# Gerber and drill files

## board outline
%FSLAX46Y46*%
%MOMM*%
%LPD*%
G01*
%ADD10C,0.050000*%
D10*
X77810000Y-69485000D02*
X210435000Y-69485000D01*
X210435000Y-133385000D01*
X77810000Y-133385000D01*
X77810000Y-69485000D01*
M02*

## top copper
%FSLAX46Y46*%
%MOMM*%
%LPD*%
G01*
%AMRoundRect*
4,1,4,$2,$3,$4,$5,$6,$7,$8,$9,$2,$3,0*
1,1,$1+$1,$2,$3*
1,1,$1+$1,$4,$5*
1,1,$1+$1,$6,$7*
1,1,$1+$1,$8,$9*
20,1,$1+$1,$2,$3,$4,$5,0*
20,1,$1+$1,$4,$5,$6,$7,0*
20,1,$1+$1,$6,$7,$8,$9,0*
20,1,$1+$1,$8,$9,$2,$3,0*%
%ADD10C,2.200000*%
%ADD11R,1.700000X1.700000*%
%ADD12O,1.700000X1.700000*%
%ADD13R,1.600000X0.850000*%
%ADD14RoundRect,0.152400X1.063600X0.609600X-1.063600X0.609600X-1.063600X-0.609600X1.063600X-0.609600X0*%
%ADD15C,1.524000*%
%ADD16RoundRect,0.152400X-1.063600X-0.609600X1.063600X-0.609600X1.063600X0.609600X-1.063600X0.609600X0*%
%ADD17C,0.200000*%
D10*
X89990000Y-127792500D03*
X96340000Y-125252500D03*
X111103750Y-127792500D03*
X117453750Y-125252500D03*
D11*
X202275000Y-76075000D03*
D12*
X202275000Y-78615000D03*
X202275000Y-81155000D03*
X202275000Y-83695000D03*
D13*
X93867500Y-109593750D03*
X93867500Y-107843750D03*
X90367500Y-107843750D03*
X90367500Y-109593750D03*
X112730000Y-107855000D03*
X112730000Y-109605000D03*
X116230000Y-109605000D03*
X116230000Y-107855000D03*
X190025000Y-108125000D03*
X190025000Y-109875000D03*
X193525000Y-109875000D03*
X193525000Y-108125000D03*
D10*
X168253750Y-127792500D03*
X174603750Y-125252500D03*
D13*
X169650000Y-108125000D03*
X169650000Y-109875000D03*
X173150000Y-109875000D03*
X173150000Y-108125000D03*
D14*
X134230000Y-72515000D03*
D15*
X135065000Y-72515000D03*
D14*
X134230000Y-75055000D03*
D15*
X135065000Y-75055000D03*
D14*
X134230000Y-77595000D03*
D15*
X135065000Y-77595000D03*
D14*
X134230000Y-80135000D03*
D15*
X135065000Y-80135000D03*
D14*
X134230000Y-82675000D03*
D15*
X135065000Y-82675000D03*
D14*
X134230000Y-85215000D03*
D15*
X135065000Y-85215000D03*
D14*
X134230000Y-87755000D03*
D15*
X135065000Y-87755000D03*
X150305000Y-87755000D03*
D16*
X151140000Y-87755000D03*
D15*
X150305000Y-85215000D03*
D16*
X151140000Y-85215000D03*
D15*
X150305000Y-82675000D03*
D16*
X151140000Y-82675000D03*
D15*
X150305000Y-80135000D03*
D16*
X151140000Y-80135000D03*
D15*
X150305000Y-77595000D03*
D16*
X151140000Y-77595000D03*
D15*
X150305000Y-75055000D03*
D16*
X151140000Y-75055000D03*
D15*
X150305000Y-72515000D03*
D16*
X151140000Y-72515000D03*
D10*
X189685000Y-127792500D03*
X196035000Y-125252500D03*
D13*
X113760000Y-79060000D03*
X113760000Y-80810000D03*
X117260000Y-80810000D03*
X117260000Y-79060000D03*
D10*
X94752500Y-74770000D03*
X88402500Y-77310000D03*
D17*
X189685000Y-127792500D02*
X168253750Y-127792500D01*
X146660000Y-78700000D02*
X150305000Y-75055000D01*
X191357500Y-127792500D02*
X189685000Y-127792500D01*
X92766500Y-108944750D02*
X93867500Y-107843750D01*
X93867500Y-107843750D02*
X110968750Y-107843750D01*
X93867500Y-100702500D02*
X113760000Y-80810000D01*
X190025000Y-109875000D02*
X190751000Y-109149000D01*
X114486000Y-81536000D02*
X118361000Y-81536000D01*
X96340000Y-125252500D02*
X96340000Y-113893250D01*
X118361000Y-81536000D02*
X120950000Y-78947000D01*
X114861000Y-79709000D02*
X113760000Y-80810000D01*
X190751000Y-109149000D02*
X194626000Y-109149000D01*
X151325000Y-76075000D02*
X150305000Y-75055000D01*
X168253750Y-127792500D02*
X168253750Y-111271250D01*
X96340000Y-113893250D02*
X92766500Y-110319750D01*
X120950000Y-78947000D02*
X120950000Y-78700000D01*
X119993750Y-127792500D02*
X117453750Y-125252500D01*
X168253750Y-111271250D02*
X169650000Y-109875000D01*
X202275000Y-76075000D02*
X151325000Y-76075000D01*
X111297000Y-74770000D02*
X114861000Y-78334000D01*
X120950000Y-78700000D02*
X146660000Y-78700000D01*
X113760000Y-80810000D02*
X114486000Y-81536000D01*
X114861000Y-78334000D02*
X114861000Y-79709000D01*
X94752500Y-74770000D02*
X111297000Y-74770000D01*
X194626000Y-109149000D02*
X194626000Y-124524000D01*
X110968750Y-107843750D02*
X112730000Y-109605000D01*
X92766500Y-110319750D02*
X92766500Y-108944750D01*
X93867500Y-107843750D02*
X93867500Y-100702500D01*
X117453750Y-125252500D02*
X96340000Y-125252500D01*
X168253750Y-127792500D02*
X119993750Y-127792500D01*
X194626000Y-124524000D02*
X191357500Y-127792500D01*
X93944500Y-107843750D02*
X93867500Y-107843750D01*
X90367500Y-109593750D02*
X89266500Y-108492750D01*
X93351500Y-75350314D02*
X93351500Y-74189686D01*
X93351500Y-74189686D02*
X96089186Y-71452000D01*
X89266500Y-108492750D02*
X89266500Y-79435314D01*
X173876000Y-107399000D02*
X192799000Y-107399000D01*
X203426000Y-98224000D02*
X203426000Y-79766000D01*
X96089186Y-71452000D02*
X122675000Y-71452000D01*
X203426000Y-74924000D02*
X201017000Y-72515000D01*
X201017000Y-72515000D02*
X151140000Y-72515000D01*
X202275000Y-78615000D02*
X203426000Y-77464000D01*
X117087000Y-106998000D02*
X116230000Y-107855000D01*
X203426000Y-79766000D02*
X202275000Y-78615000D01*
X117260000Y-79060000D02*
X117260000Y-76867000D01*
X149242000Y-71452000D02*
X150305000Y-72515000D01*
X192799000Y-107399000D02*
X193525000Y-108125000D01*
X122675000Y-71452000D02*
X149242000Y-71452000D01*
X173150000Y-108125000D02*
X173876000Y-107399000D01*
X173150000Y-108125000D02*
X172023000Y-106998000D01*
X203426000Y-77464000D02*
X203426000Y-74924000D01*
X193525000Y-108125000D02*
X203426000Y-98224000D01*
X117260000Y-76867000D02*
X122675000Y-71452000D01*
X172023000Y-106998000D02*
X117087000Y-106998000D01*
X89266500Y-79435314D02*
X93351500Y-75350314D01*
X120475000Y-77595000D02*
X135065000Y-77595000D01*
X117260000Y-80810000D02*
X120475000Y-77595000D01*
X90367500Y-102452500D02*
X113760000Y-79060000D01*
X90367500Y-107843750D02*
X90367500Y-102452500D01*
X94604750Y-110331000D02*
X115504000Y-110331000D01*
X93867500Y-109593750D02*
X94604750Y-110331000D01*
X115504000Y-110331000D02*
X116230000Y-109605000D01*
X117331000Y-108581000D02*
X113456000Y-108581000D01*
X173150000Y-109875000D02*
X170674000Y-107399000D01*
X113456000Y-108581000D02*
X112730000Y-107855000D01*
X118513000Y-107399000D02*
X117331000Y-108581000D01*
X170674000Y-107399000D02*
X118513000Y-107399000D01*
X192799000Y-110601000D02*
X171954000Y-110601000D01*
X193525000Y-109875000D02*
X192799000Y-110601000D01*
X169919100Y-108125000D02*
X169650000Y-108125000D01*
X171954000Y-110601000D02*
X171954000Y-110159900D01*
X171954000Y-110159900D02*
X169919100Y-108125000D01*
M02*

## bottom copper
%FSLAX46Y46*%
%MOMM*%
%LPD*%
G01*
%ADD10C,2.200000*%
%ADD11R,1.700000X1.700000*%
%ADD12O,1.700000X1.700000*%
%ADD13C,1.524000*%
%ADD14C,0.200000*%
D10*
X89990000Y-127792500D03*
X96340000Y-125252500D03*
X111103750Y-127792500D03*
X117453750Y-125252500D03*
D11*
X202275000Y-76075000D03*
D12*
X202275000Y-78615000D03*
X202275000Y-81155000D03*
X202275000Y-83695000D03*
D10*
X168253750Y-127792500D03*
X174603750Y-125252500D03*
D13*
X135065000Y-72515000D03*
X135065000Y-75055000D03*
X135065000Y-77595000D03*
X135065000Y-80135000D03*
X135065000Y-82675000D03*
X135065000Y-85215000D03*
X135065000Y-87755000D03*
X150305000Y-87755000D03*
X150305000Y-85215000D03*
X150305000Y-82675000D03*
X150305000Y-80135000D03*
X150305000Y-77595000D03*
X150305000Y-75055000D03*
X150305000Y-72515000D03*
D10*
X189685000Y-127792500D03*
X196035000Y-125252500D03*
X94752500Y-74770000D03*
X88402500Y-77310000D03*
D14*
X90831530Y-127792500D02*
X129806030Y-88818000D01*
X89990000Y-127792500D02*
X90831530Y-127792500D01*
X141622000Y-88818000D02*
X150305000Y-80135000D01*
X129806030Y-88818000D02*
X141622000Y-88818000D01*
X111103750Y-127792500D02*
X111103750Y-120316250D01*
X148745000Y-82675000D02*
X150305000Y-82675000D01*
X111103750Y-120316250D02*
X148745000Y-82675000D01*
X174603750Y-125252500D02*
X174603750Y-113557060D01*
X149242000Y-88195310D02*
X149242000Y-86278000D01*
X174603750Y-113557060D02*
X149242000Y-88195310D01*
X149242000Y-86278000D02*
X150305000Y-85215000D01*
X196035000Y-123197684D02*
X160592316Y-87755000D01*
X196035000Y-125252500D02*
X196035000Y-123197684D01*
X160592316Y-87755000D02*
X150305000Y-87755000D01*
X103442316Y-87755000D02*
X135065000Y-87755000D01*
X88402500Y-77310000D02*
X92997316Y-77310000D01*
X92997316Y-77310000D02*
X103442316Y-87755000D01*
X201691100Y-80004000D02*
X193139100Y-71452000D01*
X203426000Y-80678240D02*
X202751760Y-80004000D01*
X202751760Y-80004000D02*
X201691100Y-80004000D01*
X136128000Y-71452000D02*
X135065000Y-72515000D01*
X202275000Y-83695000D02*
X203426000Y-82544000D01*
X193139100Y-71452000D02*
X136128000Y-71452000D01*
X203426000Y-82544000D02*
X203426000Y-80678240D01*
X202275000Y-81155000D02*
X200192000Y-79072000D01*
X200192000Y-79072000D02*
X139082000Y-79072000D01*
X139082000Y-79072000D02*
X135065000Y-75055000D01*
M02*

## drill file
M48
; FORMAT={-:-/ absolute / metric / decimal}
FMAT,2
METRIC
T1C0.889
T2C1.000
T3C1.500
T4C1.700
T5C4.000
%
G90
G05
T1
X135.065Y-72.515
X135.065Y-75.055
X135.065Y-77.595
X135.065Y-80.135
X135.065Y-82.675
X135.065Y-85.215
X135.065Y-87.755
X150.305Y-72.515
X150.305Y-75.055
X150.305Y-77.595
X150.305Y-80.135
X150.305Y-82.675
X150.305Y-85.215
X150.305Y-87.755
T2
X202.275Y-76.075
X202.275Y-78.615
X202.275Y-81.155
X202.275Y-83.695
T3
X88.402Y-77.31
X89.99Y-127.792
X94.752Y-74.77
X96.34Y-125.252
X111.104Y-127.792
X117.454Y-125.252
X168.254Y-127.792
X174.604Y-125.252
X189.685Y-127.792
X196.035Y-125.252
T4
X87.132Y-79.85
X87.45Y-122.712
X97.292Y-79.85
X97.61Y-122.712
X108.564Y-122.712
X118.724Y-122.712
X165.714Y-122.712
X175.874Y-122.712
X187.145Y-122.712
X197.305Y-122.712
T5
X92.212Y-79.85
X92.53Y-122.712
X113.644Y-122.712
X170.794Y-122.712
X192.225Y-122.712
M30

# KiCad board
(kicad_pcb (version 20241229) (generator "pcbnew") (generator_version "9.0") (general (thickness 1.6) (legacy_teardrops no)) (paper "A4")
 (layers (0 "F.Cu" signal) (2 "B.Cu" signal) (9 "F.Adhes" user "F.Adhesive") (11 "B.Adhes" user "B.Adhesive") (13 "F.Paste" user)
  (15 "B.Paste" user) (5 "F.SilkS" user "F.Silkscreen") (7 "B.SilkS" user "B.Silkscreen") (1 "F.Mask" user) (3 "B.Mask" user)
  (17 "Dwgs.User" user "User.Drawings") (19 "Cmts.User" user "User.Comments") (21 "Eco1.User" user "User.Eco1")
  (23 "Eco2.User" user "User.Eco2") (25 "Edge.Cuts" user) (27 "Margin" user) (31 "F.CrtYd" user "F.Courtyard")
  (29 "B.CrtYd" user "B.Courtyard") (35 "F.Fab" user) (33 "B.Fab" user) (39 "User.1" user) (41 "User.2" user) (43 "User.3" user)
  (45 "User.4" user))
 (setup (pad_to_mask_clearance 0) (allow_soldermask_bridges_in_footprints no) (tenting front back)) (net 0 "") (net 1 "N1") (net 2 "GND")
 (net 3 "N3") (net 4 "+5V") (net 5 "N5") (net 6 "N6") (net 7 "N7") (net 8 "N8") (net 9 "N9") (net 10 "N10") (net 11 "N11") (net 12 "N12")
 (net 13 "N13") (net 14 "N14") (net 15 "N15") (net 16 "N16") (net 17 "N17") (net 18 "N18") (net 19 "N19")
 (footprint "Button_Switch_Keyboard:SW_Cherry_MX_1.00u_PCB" (layer "F.Cu") (at 89.99 127.7925 180)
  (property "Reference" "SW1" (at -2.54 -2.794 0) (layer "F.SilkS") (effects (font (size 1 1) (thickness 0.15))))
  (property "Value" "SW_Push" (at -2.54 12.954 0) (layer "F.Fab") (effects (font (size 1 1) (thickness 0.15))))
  (pad "" np_thru_hole circle (at -7.62 5.08 180) (size 1.7 1.7) (drill 1.7) (layers "*.Cu" "*.Mask"))
  (pad "" np_thru_hole circle (at -2.54 5.08 180) (size 4 4) (drill 4) (layers "*.Cu" "*.Mask"))
  (pad "" np_thru_hole circle (at 2.54 5.08 180) (size 1.7 1.7) (drill 1.7) (layers "*.Cu" "*.Mask"))
  (pad "1" thru_hole circle (at 0 0 180) (size 2.2 2.2) (drill 1.5) (layers "*.Cu" "*.Mask") (remove_unused_layers no) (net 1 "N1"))
  (pad "2" thru_hole circle (at -6.35 2.54 180) (size 2.2 2.2) (drill 1.5) (layers "*.Cu" "*.Mask") (remove_unused_layers no) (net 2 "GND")))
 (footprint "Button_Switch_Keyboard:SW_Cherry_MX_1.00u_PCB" (layer "F.Cu") (at 111.10375 127.7925 180)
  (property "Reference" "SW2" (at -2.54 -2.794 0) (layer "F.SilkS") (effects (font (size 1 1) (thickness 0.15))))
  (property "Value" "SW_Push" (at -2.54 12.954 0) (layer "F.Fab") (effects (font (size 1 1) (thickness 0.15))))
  (pad "" np_thru_hole circle (at -7.62 5.08 180) (size 1.7 1.7) (drill 1.7) (layers "*.Cu" "*.Mask"))
  (pad "" np_thru_hole circle (at -2.54 5.08 180) (size 4 4) (drill 4) (layers "*.Cu" "*.Mask"))
  (pad "" np_thru_hole circle (at 2.54 5.08 180) (size 1.7 1.7) (drill 1.7) (layers "*.Cu" "*.Mask"))
  (pad "1" thru_hole circle (at 0 0 180) (size 2.2 2.2) (drill 1.5) (layers "*.Cu" "*.Mask") (remove_unused_layers no) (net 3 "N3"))
  (pad "2" thru_hole circle (at -6.35 2.54 180) (size 2.2 2.2) (drill 1.5) (layers "*.Cu" "*.Mask") (remove_unused_layers no) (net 2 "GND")))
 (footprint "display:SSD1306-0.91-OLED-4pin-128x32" (layer "F.Cu") (at 165.775 73.885)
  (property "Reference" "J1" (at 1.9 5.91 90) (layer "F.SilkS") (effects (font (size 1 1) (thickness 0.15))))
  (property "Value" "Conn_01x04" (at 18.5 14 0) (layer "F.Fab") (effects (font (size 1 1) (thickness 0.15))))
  (pad "1" thru_hole rect (at 36.5 2.19) (size 1.7 1.7) (drill 1) (layers "*.Cu" "*.Mask") (remove_unused_layers no) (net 2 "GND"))
  (pad "2" thru_hole oval (at 36.5 4.73) (size 1.7 1.7) (drill 1) (layers "*.Cu" "*.Mask") (remove_unused_layers no) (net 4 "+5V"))
  (pad "3" thru_hole oval (at 36.5 7.27) (size 1.7 1.7) (drill 1) (layers "*.Cu" "*.Mask") (remove_unused_layers no) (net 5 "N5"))
  (pad "4" thru_hole oval (at 36.5 9.81) (size 1.7 1.7) (drill 1) (layers "*.Cu" "*.Mask") (remove_unused_layers no) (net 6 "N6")))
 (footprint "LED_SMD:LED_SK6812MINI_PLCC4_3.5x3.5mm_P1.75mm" (layer "F.Cu") (at 92.1175 108.71875 180)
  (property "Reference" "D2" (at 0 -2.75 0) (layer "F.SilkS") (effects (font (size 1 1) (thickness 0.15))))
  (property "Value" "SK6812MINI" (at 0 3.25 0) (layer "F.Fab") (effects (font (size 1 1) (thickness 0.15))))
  (pad "1" smd rect (at -1.75 -0.875 180) (size 1.6 0.85) (layers "F.Cu" "F.Mask" "F.Paste") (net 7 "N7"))
  (pad "2" smd rect (at -1.75 0.875 180) (size 1.6 0.85) (layers "F.Cu" "F.Mask" "F.Paste") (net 2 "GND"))
  (pad "3" smd rect (at 1.75 0.875 180) (size 1.6 0.85) (layers "F.Cu" "F.Mask" "F.Paste") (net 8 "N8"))
  (pad "4" smd rect (at 1.75 -0.875 180) (size 1.6 0.85) (layers "F.Cu" "F.Mask" "F.Paste") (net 4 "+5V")))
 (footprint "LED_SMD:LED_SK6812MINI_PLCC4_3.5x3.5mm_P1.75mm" (layer "F.Cu") (at 114.48 108.73)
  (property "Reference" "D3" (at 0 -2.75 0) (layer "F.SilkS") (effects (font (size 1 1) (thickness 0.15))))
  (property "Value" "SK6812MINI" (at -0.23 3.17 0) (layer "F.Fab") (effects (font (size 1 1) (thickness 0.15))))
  (pad "1" smd rect (at -1.75 -0.875) (size 1.6 0.85) (layers "F.Cu" "F.Mask" "F.Paste") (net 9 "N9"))
  (pad "2" smd rect (at -1.75 0.875) (size 1.6 0.85) (layers "F.Cu" "F.Mask" "F.Paste") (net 2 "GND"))
  (pad "3" smd rect (at 1.75 0.875) (size 1.6 0.85) (layers "F.Cu" "F.Mask" "F.Paste") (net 7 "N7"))
  (pad "4" smd rect (at 1.75 -0.875) (size 1.6 0.85) (layers "F.Cu" "F.Mask" "F.Paste") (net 4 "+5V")))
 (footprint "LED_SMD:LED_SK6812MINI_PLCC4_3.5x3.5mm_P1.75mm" (layer "F.Cu") (at 191.775 109)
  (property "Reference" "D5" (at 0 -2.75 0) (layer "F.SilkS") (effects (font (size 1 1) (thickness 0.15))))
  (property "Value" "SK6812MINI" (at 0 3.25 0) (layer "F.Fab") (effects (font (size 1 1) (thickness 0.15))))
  (pad "1" smd rect (at -1.75 -0.875) (size 1.6 0.85) (layers "F.Cu" "F.Mask" "F.Paste") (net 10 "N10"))
  (pad "2" smd rect (at -1.75 0.875) (size 1.6 0.85) (layers "F.Cu" "F.Mask" "F.Paste") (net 2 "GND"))
  (pad "3" smd rect (at 1.75 0.875) (size 1.6 0.85) (layers "F.Cu" "F.Mask" "F.Paste") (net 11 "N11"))
  (pad "4" smd rect (at 1.75 -0.875) (size 1.6 0.85) (layers "F.Cu" "F.Mask" "F.Paste") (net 4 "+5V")))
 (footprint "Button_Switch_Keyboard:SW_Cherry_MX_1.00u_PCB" (layer "F.Cu") (at 168.25375 127.7925 180)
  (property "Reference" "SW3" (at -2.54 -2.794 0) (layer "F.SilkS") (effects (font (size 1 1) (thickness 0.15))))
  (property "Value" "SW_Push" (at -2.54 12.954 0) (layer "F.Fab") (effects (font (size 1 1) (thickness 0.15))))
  (pad "" np_thru_hole circle (at -7.62 5.08 180) (size 1.7 1.7) (drill 1.7) (layers "*.Cu" "*.Mask"))
  (pad "" np_thru_hole circle (at -2.54 5.08 180) (size 4 4) (drill 4) (layers "*.Cu" "*.Mask"))
  (pad "" np_thru_hole circle (at 2.54 5.08 180) (size 1.7 1.7) (drill 1.7) (layers "*.Cu" "*.Mask"))
  (pad "1" thru_hole circle (at 0 0 180) (size 2.2 2.2) (drill 1.5) (layers "*.Cu" "*.Mask") (remove_unused_layers no) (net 2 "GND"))
  (pad "2" thru_hole circle (at -6.35 2.54 180) (size 2.2 2.2) (drill 1.5) (layers "*.Cu" "*.Mask") (remove_unused_layers no) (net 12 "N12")))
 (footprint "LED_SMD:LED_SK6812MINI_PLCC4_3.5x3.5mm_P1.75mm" (layer "F.Cu") (at 171.4 109)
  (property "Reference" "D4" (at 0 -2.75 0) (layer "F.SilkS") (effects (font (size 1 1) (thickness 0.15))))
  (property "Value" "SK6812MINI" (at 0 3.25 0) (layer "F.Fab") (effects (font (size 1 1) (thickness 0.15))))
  (pad "1" smd rect (at -1.75 -0.875) (size 1.6 0.85) (layers "F.Cu" "F.Mask" "F.Paste") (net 11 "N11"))
  (pad "2" smd rect (at -1.75 0.875) (size 1.6 0.85) (layers "F.Cu" "F.Mask" "F.Paste") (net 2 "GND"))
  (pad "3" smd rect (at 1.75 0.875) (size 1.6 0.85) (layers "F.Cu" "F.Mask" "F.Paste") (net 9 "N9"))
  (pad "4" smd rect (at 1.75 -0.875) (size 1.6 0.85) (layers "F.Cu" "F.Mask" "F.Paste") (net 4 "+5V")))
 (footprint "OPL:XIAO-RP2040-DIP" (layer "F.Cu") (at 142.685 80.135)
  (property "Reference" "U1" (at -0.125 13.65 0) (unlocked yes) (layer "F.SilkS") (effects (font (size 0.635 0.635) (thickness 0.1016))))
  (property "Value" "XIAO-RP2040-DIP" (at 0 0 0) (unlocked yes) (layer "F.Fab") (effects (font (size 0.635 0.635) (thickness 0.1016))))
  (pad "1" smd roundrect (at -8.455 -7.62 180) (size 2.432 1.524) (layers "F.Cu" "F.Mask") (roundrect_rratio 0.1) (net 6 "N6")
   (thermal_bridge_angle 45))
  (pad "1" thru_hole circle (at -7.62 -7.62 180) (size 1.524 1.524) (drill 0.889) (layers "*.Cu" "*.Mask") (remove_unused_layers no)
   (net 6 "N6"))
  (pad "2" smd roundrect (at -8.455 -5.08 180) (size 2.432 1.524) (layers "F.Cu" "F.Mask") (roundrect_rratio 0.1) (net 5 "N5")
   (thermal_bridge_angle 45))
  (pad "2" thru_hole circle (at -7.62 -5.08 180) (size 1.524 1.524) (drill 0.889) (layers "*.Cu" "*.Mask") (remove_unused_layers no)
   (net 5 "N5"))
  (pad "3" smd roundrect (at -8.455 -2.54 180) (size 2.432 1.524) (layers "F.Cu" "F.Mask") (roundrect_rratio 0.1) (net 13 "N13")
   (thermal_bridge_angle 45))
  (pad "3" thru_hole circle (at -7.62 -2.54 180) (size 1.524 1.524) (drill 0.889) (layers "*.Cu" "*.Mask") (remove_unused_layers no)
   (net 13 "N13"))
  (pad "4" smd roundrect (at -8.455 0 180) (size 2.432 1.524) (layers "F.Cu" "F.Mask") (roundrect_rratio 0.1) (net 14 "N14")
   (thermal_bridge_angle 45))
  (pad "4" thru_hole circle (at -7.62 0 180) (size 1.524 1.524) (drill 0.889) (layers "*.Cu" "*.Mask") (remove_unused_layers no)
   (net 14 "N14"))
  (pad "5" smd roundrect (at -8.455 2.54 180) (size 2.432 1.524) (layers "F.Cu" "F.Mask") (roundrect_rratio 0.1) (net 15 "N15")
   (thermal_bridge_angle 45))
  (pad "5" thru_hole circle (at -7.62 2.54 180) (size 1.524 1.524) (drill 0.889) (layers "*.Cu" "*.Mask") (remove_unused_layers no)
   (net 15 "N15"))
  (pad "6" smd roundrect (at -8.455 5.08 180) (size 2.432 1.524) (layers "F.Cu" "F.Mask") (roundrect_rratio 0.1) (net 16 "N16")
   (thermal_bridge_angle 45))
  (pad "6" thru_hole circle (at -7.62 5.08 180) (size 1.524 1.524) (drill 0.889) (layers "*.Cu" "*.Mask") (remove_unused_layers no)
   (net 16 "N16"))
  (pad "7" smd roundrect (at -8.455 7.62 180) (size 2.432 1.524) (layers "F.Cu" "F.Mask") (roundrect_rratio 0.1) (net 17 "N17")
   (thermal_bridge_angle 45))
  (pad "7" thru_hole circle (at -7.62 7.62 180) (size 1.524 1.524) (drill 0.889) (layers "*.Cu" "*.Mask") (remove_unused_layers no)
   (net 17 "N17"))
  (pad "8" thru_hole circle (at 7.62 7.62) (size 1.524 1.524) (drill 0.889) (layers "*.Cu" "*.Mask") (remove_unused_layers no)
   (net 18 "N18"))
  (pad "8" smd roundrect (at 8.455 7.62) (size 2.432 1.524) (layers "F.Cu" "F.Mask") (roundrect_rratio 0.1) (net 18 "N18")
   (thermal_bridge_angle 45))
  (pad "9" thru_hole circle (at 7.62 5.08) (size 1.524 1.524) (drill 0.889) (layers "*.Cu" "*.Mask") (remove_unused_layers no)
   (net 12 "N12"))
  (pad "9" smd roundrect (at 8.455 5.08) (size 2.432 1.524) (layers "F.Cu" "F.Mask") (roundrect_rratio 0.1) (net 12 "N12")
   (thermal_bridge_angle 45))
  (pad "10" thru_hole circle (at 7.62 2.54) (size 1.524 1.524) (drill 0.889) (layers "*.Cu" "*.Mask") (remove_unused_layers no) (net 3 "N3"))
  (pad "10" smd roundrect (at 8.455 2.54) (size 2.432 1.524) (layers "F.Cu" "F.Mask") (roundrect_rratio 0.1) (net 3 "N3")
   (thermal_bridge_angle 45))
  (pad "11" thru_hole circle (at 7.62 0) (size 1.524 1.524) (drill 0.889) (layers "*.Cu" "*.Mask") (remove_unused_layers no) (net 1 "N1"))
  (pad "11" smd roundrect (at 8.455 0) (size 2.432 1.524) (layers "F.Cu" "F.Mask") (roundrect_rratio 0.1) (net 1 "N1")
   (thermal_bridge_angle 45))
  (pad "12" thru_hole circle (at 7.62 -2.54) (size 1.524 1.524) (drill 0.889) (layers "*.Cu" "*.Mask") (remove_unused_layers no)
   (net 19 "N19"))
  (pad "12" smd roundrect (at 8.455 -2.54) (size 2.432 1.524) (layers "F.Cu" "F.Mask") (roundrect_rratio 0.1) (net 19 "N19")
   (thermal_bridge_angle 45))
  (pad "13" thru_hole circle (at 7.62 -5.08) (size 1.524 1.524) (drill 0.889) (layers "*.Cu" "*.Mask") (remove_unused_layers no)
   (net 2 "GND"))
  (pad "13" smd roundrect (at 8.455 -5.08) (size 2.432 1.524) (layers "F.Cu" "F.Mask") (roundrect_rratio 0.1) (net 2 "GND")
   (thermal_bridge_angle 45))
  (pad "14" thru_hole circle (at 7.62 -7.62) (size 1.524 1.524) (drill 0.889) (layers "*.Cu" "*.Mask") (remove_unused_layers no)
   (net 4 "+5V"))
  (pad "14" smd roundrect (at 8.455 -7.62) (size 2.432 1.524) (layers "F.Cu" "F.Mask") (roundrect_rratio 0.1) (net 4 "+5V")
   (thermal_bridge_angle 45)))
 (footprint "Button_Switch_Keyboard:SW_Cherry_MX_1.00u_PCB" (layer "F.Cu") (at 189.685 127.7925 180)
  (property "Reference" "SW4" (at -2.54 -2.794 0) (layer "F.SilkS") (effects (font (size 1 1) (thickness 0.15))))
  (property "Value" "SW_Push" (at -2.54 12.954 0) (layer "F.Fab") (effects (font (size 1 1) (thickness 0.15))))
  (pad "" np_thru_hole circle (at -7.62 5.08 180) (size 1.7 1.7) (drill 1.7) (layers "*.Cu" "*.Mask"))
  (pad "" np_thru_hole circle (at -2.54 5.08 180) (size 4 4) (drill 4) (layers "*.Cu" "*.Mask"))
  (pad "" np_thru_hole circle (at 2.54 5.08 180) (size 1.7 1.7) (drill 1.7) (layers "*.Cu" "*.Mask"))
  (pad "1" thru_hole circle (at 0 0 180) (size 2.2 2.2) (drill 1.5) (layers "*.Cu" "*.Mask") (remove_unused_layers no) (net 2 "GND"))
  (pad "2" thru_hole circle (at -6.35 2.54 180) (size 2.2 2.2) (drill 1.5) (layers "*.Cu" "*.Mask") (remove_unused_layers no) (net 18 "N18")))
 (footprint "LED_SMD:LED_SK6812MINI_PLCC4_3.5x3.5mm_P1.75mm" (layer "F.Cu") (at 115.51 79.935)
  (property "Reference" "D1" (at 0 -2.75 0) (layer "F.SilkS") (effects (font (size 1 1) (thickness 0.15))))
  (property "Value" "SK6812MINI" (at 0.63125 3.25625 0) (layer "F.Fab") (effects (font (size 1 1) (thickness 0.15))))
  (pad "1" smd rect (at -1.75 -0.875) (size 1.6 0.85) (layers "F.Cu" "F.Mask" "F.Paste") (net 8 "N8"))
  (pad "2" smd rect (at -1.75 0.875) (size 1.6 0.85) (layers "F.Cu" "F.Mask" "F.Paste") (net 2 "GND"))
  (pad "3" smd rect (at 1.75 0.875) (size 1.6 0.85) (layers "F.Cu" "F.Mask" "F.Paste") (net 13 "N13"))
  (pad "4" smd rect (at 1.75 -0.875) (size 1.6 0.85) (layers "F.Cu" "F.Mask" "F.Paste") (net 4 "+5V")))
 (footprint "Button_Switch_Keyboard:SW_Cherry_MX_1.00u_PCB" (layer "F.Cu") (at 94.7525 74.77)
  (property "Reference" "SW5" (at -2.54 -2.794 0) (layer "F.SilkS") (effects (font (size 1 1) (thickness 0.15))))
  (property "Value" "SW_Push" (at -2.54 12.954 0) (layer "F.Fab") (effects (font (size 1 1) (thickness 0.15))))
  (pad "" np_thru_hole circle (at -7.62 5.08) (size 1.7 1.7) (drill 1.7) (layers "*.Cu" "*.Mask"))
  (pad "" np_thru_hole circle (at -2.54 5.08) (size 4 4) (drill 4) (layers "*.Cu" "*.Mask"))
  (pad "" np_thru_hole circle (at 2.54 5.08) (size 1.7 1.7) (drill 1.7) (layers "*.Cu" "*.Mask"))
  (pad "1" thru_hole circle (at 0 0) (size 2.2 2.2) (drill 1.5) (layers "*.Cu" "*.Mask") (remove_unused_layers no) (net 2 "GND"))
  (pad "2" thru_hole circle (at -6.35 2.54) (size 2.2 2.2) (drill 1.5) (layers "*.Cu" "*.Mask") (remove_unused_layers no) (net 17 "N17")))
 (gr_rect (start 77.81 69.485) (end 210.435 133.385) (stroke (width 0.05) (type default)) (fill no) (layer "Edge.Cuts"))
 (segment (start 189.685 127.7925) (end 168.25375 127.7925) (width 0.2) (layer "F.Cu") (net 2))
 (segment (start 146.66 78.7) (end 150.305 75.055) (width 0.2) (layer "F.Cu") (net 2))
 (segment (start 191.3575 127.7925) (end 189.685 127.7925) (width 0.2) (layer "F.Cu") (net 2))
 (segment (start 92.7665 108.94475) (end 93.8675 107.84375) (width 0.2) (layer "F.Cu") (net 2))
 (segment (start 93.8675 107.84375) (end 110.96875 107.84375) (width 0.2) (layer "F.Cu") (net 2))
 (segment (start 93.8675 100.7025) (end 113.76 80.81) (width 0.2) (layer "F.Cu") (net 2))
 (segment (start 190.025 109.875) (end 190.751 109.149) (width 0.2) (layer "F.Cu") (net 2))
 (segment (start 114.486 81.536) (end 118.361 81.536) (width 0.2) (layer "F.Cu") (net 2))
 (segment (start 96.34 125.2525) (end 96.34 113.89325) (width 0.2) (layer "F.Cu") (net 2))
 (segment (start 118.361 81.536) (end 120.95 78.947) (width 0.2) (layer "F.Cu") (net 2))
 (segment (start 114.861 79.709) (end 113.76 80.81) (width 0.2) (layer "F.Cu") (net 2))
 (segment (start 190.751 109.149) (end 194.626 109.149) (width 0.2) (layer "F.Cu") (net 2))
 (segment (start 151.325 76.075) (end 150.305 75.055) (width 0.2) (layer "F.Cu") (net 2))
 (segment (start 168.25375 127.7925) (end 168.25375 111.27125) (width 0.2) (layer "F.Cu") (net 2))
 (segment (start 96.34 113.89325) (end 92.7665 110.31975) (width 0.2) (layer "F.Cu") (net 2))
 (segment (start 120.95 78.947) (end 120.95 78.7) (width 0.2) (layer "F.Cu") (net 2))
 (segment (start 119.99375 127.7925) (end 117.45375 125.2525) (width 0.2) (layer "F.Cu") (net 2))
 (segment (start 168.25375 111.27125) (end 169.65 109.875) (width 0.2) (layer "F.Cu") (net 2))
 (segment (start 202.275 76.075) (end 151.325 76.075) (width 0.2) (layer "F.Cu") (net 2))
 (segment (start 111.297 74.77) (end 114.861 78.334) (width 0.2) (layer "F.Cu") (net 2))
 (segment (start 120.95 78.7) (end 146.66 78.7) (width 0.2) (layer "F.Cu") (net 2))
 (segment (start 113.76 80.81) (end 114.486 81.536) (width 0.2) (layer "F.Cu") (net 2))
 (segment (start 114.861 78.334) (end 114.861 79.709) (width 0.2) (layer "F.Cu") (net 2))
 (segment (start 94.7525 74.77) (end 111.297 74.77) (width 0.2) (layer "F.Cu") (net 2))
 (segment (start 194.626 109.149) (end 194.626 124.524) (width 0.2) (layer "F.Cu") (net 2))
 (segment (start 110.96875 107.84375) (end 112.73 109.605) (width 0.2) (layer "F.Cu") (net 2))
 (segment (start 92.7665 110.31975) (end 92.7665 108.94475) (width 0.2) (layer "F.Cu") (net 2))
 (segment (start 93.8675 107.84375) (end 93.8675 100.7025) (width 0.2) (layer "F.Cu") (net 2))
 (segment (start 117.45375 125.2525) (end 96.34 125.2525) (width 0.2) (layer "F.Cu") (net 2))
 (segment (start 168.25375 127.7925) (end 119.99375 127.7925) (width 0.2) (layer "F.Cu") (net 2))
 (segment (start 194.626 124.524) (end 191.3575 127.7925) (width 0.2) (layer "F.Cu") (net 2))
 (segment (start 93.9445 107.84375) (end 93.8675 107.84375) (width 0.2) (layer "F.Cu") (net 2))
 (segment (start 90.3675 109.59375) (end 89.2665 108.49275) (width 0.2) (layer "F.Cu") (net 4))
 (segment (start 93.3515 75.350314) (end 93.3515 74.189686) (width 0.2) (layer "F.Cu") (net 4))
 (segment (start 93.3515 74.189686) (end 96.089186 71.452) (width 0.2) (layer "F.Cu") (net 4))
 (segment (start 89.2665 108.49275) (end 89.2665 79.435314) (width 0.2) (layer "F.Cu") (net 4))
 (segment (start 173.876 107.399) (end 192.799 107.399) (width 0.2) (layer "F.Cu") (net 4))
 (segment (start 203.426 98.224) (end 203.426 79.766) (width 0.2) (layer "F.Cu") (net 4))
 (segment (start 96.089186 71.452) (end 122.675 71.452) (width 0.2) (layer "F.Cu") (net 4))
 (segment (start 203.426 74.924) (end 201.017 72.515) (width 0.2) (layer "F.Cu") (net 4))
 (segment (start 201.017 72.515) (end 151.14 72.515) (width 0.2) (layer "F.Cu") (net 4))
 (segment (start 202.275 78.615) (end 203.426 77.464) (width 0.2) (layer "F.Cu") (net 4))
 (segment (start 117.087 106.998) (end 116.23 107.855) (width 0.2) (layer "F.Cu") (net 4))
 (segment (start 203.426 79.766) (end 202.275 78.615) (width 0.2) (layer "F.Cu") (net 4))
 (segment (start 117.26 79.06) (end 117.26 76.867) (width 0.2) (layer "F.Cu") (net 4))
 (segment (start 149.242 71.452) (end 150.305 72.515) (width 0.2) (layer "F.Cu") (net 4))
 (segment (start 192.799 107.399) (end 193.525 108.125) (width 0.2) (layer "F.Cu") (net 4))
 (segment (start 122.675 71.452) (end 149.242 71.452) (width 0.2) (layer "F.Cu") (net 4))
 (segment (start 173.15 108.125) (end 173.876 107.399) (width 0.2) (layer "F.Cu") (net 4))
 (segment (start 173.15 108.125) (end 172.023 106.998) (width 0.2) (layer "F.Cu") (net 4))
 (segment (start 203.426 77.464) (end 203.426 74.924) (width 0.2) (layer "F.Cu") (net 4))
 (segment (start 193.525 108.125) (end 203.426 98.224) (width 0.2) (layer "F.Cu") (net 4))
 (segment (start 117.26 76.867) (end 122.675 71.452) (width 0.2) (layer "F.Cu") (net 4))
 (segment (start 172.023 106.998) (end 117.087 106.998) (width 0.2) (layer "F.Cu") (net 4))
 (segment (start 89.2665 79.435314) (end 93.3515 75.350314) (width 0.2) (layer "F.Cu") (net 4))
 (segment (start 120.475 77.595) (end 135.065 77.595) (width 0.2) (layer "F.Cu") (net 13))
 (segment (start 117.26 80.81) (end 120.475 77.595) (width 0.2) (layer "F.Cu") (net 13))
 (segment (start 90.3675 102.4525) (end 113.76 79.06) (width 0.2) (layer "F.Cu") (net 8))
 (segment (start 90.3675 107.84375) (end 90.3675 102.4525) (width 0.2) (layer "F.Cu") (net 8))
 (segment (start 94.60475 110.331) (end 115.504 110.331) (width 0.2) (layer "F.Cu") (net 7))
 (segment (start 93.8675 109.59375) (end 94.60475 110.331) (width 0.2) (layer "F.Cu") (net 7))
 (segment (start 115.504 110.331) (end 116.23 109.605) (width 0.2) (layer "F.Cu") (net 7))
 (segment (start 90.83153 127.7925) (end 129.80603 88.818) (width 0.2) (layer "B.Cu") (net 1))
 (segment (start 89.99 127.7925) (end 90.83153 127.7925) (width 0.2) (layer "B.Cu") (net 1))
 (segment (start 141.622 88.818) (end 150.305 80.135) (width 0.2) (layer "B.Cu") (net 1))
 (segment (start 129.80603 88.818) (end 141.622 88.818) (width 0.2) (layer "B.Cu") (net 1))
 (segment (start 111.10375 127.7925) (end 111.10375 120.31625) (width 0.2) (layer "B.Cu") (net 3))
 (segment (start 148.745 82.675) (end 150.305 82.675) (width 0.2) (layer "B.Cu") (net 3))
 (segment (start 111.10375 120.31625) (end 148.745 82.675) (width 0.2) (layer "B.Cu") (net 3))
 (segment (start 174.60375 125.2525) (end 174.60375 113.55706) (width 0.2) (layer "B.Cu") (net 12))
 (segment (start 149.242 88.19531) (end 149.242 86.278) (width 0.2) (layer "B.Cu") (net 12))
 (segment (start 174.60375 113.55706) (end 149.242 88.19531) (width 0.2) (layer "B.Cu") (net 12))
 (segment (start 149.242 86.278) (end 150.305 85.215) (width 0.2) (layer "B.Cu") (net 12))
 (segment (start 196.035 123.197684) (end 160.592316 87.755) (width 0.2) (layer "B.Cu") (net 18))
 (segment (start 196.035 125.2525) (end 196.035 123.197684) (width 0.2) (layer "B.Cu") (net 18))
 (segment (start 160.592316 87.755) (end 150.305 87.755) (width 0.2) (layer "B.Cu") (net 18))
 (segment (start 103.442316 87.755) (end 135.065 87.755) (width 0.2) (layer "B.Cu") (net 17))
 (segment (start 88.4025 77.31) (end 92.997316 77.31) (width 0.2) (layer "B.Cu") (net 17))
 (segment (start 92.997316 77.31) (end 103.442316 87.755) (width 0.2) (layer "B.Cu") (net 17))
 (segment (start 117.331 108.581) (end 113.456 108.581) (width 0.2) (layer "F.Cu") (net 9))
 (segment (start 173.15 109.875) (end 170.674 107.399) (width 0.2) (layer "F.Cu") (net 9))
 (segment (start 113.456 108.581) (end 112.73 107.855) (width 0.2) (layer "F.Cu") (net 9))
 (segment (start 118.513 107.399) (end 117.331 108.581) (width 0.2) (layer "F.Cu") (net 9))
 (segment (start 170.674 107.399) (end 118.513 107.399) (width 0.2) (layer "F.Cu") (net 9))
 (segment (start 192.799 110.601) (end 171.954 110.601) (width 0.2) (layer "F.Cu") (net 11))
 (segment (start 193.525 109.875) (end 192.799 110.601) (width 0.2) (layer "F.Cu") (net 11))
 (segment (start 169.9191 108.125) (end 169.65 108.125) (width 0.2) (layer "F.Cu") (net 11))
 (segment (start 171.954 110.601) (end 171.954 110.1599) (width 0.2) (layer "F.Cu") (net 11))
 (segment (start 171.954 110.1599) (end 169.9191 108.125) (width 0.2) (layer "F.Cu") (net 11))
 (segment (start 201.6911 80.004) (end 193.1391 71.452) (width 0.2) (layer "B.Cu") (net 6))
 (segment (start 203.426 80.67824) (end 202.75176 80.004) (width 0.2) (layer "B.Cu") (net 6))
 (segment (start 202.75176 80.004) (end 201.6911 80.004) (width 0.2) (layer "B.Cu") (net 6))
 (segment (start 136.128 71.452) (end 135.065 72.515) (width 0.2) (layer "B.Cu") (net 6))
 (segment (start 202.275 83.695) (end 203.426 82.544) (width 0.2) (layer "B.Cu") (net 6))
 (segment (start 193.1391 71.452) (end 136.128 71.452) (width 0.2) (layer "B.Cu") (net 6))
 (segment (start 203.426 82.544) (end 203.426 80.67824) (width 0.2) (layer "B.Cu") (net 6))
 (segment (start 202.275 81.155) (end 200.192 79.072) (width 0.2) (layer "B.Cu") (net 5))
 (segment (start 200.192 79.072) (end 139.082 79.072) (width 0.2) (layer "B.Cu") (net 5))
 (segment (start 139.082 79.072) (end 135.065 75.055) (width 0.2) (layer "B.Cu") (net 5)))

